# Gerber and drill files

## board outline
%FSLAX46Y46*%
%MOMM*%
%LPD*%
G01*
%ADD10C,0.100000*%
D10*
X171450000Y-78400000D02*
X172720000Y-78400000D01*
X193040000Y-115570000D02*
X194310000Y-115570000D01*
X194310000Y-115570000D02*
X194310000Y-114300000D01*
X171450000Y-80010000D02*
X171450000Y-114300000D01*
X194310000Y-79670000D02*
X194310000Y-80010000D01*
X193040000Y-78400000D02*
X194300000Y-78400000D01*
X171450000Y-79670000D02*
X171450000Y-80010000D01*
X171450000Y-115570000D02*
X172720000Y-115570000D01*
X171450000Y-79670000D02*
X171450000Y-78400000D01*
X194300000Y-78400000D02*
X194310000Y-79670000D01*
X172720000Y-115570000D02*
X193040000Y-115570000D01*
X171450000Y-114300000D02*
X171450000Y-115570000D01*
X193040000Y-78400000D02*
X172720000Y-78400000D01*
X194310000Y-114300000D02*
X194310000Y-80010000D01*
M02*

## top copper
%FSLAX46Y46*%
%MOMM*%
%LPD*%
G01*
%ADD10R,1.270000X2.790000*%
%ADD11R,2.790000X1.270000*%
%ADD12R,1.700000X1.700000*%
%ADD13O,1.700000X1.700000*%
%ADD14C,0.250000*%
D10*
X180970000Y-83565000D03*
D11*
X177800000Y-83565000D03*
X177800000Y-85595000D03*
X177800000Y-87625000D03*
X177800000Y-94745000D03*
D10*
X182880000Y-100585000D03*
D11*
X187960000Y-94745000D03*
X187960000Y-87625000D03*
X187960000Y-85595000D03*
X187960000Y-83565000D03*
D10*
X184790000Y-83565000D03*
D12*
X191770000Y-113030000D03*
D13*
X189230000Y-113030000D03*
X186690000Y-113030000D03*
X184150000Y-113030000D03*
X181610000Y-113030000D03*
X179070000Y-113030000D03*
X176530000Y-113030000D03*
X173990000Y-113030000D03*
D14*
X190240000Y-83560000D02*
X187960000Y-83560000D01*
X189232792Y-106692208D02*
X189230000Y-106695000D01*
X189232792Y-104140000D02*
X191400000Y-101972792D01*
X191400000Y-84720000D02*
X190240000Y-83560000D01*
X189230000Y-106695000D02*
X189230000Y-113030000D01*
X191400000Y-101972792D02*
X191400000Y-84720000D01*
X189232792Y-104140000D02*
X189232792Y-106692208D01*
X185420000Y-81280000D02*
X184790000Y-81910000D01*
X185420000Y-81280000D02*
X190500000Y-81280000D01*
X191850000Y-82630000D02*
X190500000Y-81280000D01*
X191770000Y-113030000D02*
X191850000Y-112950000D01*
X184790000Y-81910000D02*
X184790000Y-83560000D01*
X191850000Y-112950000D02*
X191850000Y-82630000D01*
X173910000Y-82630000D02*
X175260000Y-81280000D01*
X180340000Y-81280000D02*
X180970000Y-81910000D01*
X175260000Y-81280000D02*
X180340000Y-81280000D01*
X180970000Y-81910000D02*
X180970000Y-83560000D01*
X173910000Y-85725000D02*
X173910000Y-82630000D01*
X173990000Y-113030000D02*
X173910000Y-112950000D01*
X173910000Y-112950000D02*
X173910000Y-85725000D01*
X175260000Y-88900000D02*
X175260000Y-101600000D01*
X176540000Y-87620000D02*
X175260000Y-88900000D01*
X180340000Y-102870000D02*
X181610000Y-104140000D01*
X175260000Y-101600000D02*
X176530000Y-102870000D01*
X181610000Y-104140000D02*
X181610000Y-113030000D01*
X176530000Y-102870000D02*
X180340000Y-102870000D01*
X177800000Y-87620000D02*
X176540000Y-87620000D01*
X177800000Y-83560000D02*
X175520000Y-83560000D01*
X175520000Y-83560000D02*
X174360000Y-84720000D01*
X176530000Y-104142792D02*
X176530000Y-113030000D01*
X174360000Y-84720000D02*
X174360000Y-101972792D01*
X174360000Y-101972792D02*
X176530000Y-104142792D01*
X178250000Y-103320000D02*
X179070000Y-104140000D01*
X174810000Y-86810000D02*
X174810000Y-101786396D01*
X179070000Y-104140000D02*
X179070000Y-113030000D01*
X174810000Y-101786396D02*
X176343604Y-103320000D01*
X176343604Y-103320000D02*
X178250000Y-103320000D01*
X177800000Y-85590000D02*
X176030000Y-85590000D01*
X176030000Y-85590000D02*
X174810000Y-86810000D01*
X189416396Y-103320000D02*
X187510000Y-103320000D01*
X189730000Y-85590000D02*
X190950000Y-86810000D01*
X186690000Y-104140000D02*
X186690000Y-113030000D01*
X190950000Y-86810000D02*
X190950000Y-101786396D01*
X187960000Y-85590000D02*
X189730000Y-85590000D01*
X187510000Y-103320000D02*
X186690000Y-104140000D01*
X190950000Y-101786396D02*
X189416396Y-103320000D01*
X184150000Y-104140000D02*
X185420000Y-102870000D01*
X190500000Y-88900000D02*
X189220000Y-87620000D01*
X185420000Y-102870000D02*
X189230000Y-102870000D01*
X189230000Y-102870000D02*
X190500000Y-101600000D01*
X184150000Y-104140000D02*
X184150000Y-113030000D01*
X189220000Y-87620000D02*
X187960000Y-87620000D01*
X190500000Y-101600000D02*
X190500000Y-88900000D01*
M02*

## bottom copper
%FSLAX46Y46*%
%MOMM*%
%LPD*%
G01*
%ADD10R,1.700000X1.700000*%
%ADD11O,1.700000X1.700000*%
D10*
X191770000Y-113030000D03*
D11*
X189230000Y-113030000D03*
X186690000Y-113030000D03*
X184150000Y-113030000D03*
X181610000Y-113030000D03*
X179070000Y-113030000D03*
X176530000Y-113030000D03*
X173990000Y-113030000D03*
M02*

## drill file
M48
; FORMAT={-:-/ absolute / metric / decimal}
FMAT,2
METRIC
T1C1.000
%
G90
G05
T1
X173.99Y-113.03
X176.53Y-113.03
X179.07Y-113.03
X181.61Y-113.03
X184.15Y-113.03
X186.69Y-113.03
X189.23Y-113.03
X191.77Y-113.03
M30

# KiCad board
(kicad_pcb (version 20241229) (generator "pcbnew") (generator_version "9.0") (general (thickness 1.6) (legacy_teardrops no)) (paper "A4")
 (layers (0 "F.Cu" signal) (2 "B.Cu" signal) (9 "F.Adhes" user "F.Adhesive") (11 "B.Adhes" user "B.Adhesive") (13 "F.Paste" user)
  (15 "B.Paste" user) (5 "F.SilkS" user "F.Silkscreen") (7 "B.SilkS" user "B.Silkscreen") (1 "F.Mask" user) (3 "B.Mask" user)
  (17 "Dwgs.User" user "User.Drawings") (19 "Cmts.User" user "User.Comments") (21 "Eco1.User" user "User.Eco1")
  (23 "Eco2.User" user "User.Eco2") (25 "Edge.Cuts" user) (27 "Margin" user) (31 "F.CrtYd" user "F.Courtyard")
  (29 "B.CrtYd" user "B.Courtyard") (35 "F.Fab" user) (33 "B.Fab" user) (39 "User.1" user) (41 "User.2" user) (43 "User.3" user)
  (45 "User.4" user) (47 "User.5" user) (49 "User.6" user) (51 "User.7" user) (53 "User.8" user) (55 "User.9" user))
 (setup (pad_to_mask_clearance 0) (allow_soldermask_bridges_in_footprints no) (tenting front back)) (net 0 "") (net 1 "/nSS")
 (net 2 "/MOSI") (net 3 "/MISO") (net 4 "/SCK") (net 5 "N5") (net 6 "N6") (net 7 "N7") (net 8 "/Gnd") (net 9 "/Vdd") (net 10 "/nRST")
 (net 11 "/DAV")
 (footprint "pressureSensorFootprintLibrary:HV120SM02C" (layer "F.Cu") (at 182.88 92.075 90)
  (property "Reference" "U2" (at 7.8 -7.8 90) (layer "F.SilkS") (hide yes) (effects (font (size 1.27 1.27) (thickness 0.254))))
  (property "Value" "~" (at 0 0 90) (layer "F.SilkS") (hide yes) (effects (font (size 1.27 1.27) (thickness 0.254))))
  (pad "1" smd rect (at 8.51 -1.91 180) (size 1.27 2.79) (layers "F.Cu" "F.Mask" "F.Paste") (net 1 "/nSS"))
  (pad "2" smd rect (at 8.51 -5.08 90) (size 1.27 2.79) (layers "F.Cu" "F.Mask" "F.Paste") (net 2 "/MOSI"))
  (pad "3" smd rect (at 6.48 -5.08 90) (size 1.27 2.79) (layers "F.Cu" "F.Mask" "F.Paste") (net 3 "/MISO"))
  (pad "4" smd rect (at 4.45 -5.08 90) (size 1.27 2.79) (layers "F.Cu" "F.Mask" "F.Paste") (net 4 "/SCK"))
  (pad "5" smd rect (at -2.67 -5.08 90) (size 1.27 2.79) (layers "F.Cu" "F.Mask" "F.Paste") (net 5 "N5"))
  (pad "6" smd rect (at -8.51 0 180) (size 1.27 2.79) (layers "F.Cu" "F.Mask" "F.Paste") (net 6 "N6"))
  (pad "7" smd rect (at -2.67 5.08 90) (size 1.27 2.79) (layers "F.Cu" "F.Mask" "F.Paste") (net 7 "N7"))
  (pad "8" smd rect (at 4.45 5.08 90) (size 1.27 2.79) (layers "F.Cu" "F.Mask" "F.Paste") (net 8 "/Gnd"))
  (pad "9" smd rect (at 6.48 5.08 90) (size 1.27 2.79) (layers "F.Cu" "F.Mask" "F.Paste") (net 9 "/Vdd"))
  (pad "10" smd rect (at 8.51 5.08 90) (size 1.27 2.79) (layers "F.Cu" "F.Mask" "F.Paste") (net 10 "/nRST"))
  (pad "11" smd rect (at 8.51 1.91 180) (size 1.27 2.79) (layers "F.Cu" "F.Mask" "F.Paste") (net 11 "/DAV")))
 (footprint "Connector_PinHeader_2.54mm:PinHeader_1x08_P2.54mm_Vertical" (layer "B.Cu") (at 191.77 113.03 90)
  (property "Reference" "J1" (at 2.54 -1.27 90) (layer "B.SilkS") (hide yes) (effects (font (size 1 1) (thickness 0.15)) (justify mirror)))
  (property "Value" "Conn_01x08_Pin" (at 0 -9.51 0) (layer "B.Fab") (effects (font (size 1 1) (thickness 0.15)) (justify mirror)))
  (pad "1" thru_hole rect (at 0 0 90) (size 1.7 1.7) (drill 1) (layers "*.Cu" "*.Mask") (remove_unused_layers no) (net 11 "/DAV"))
  (pad "2" thru_hole oval (at 0 -2.54 90) (size 1.7 1.7) (drill 1) (layers "*.Cu" "*.Mask") (remove_unused_layers no) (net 10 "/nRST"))
  (pad "3" thru_hole oval (at 0 -5.08 90) (size 1.7 1.7) (drill 1) (layers "*.Cu" "*.Mask") (remove_unused_layers no) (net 9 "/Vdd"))
  (pad "4" thru_hole oval (at 0 -7.62 90) (size 1.7 1.7) (drill 1) (layers "*.Cu" "*.Mask") (remove_unused_layers no) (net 8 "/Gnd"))
  (pad "5" thru_hole oval (at 0 -10.16 90) (size 1.7 1.7) (drill 1) (layers "*.Cu" "*.Mask") (remove_unused_layers no) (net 4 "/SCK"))
  (pad "6" thru_hole oval (at 0 -12.7 90) (size 1.7 1.7) (drill 1) (layers "*.Cu" "*.Mask") (remove_unused_layers no) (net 3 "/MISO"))
  (pad "7" thru_hole oval (at 0 -15.24 90) (size 1.7 1.7) (drill 1) (layers "*.Cu" "*.Mask") (remove_unused_layers no) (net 2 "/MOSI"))
  (pad "8" thru_hole oval (at 0 -17.78 90) (size 1.7 1.7) (drill 1) (layers "*.Cu" "*.Mask") (remove_unused_layers no) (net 1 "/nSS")))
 (gr_line (start 171.45 78.4) (end 172.72 78.4) (stroke (width 0.1) (type default)) (layer "Edge.Cuts"))
 (gr_line (start 193.04 115.57) (end 194.31 115.57) (stroke (width 0.1) (type default)) (layer "Edge.Cuts"))
 (gr_line (start 194.31 115.57) (end 194.31 114.3) (stroke (width 0.1) (type default)) (layer "Edge.Cuts"))
 (gr_line (start 171.45 80.01) (end 171.45 114.3) (stroke (width 0.1) (type default)) (layer "Edge.Cuts"))
 (gr_line (start 194.31 79.67) (end 194.31 80.01) (stroke (width 0.1) (type default)) (layer "Edge.Cuts"))
 (gr_line (start 193.04 78.4) (end 194.3 78.4) (stroke (width 0.1) (type default)) (layer "Edge.Cuts"))
 (gr_line (start 171.45 79.67) (end 171.45 80.01) (stroke (width 0.1) (type default)) (layer "Edge.Cuts"))
 (gr_line (start 171.45 115.57) (end 172.72 115.57) (stroke (width 0.1) (type default)) (layer "Edge.Cuts"))
 (gr_line (start 171.45 79.67) (end 171.45 78.4) (stroke (width 0.1) (type default)) (layer "Edge.Cuts"))
 (gr_line (start 194.3 78.4) (end 194.31 79.67) (stroke (width 0.1) (type default)) (layer "Edge.Cuts"))
 (gr_line (start 172.72 115.57) (end 193.04 115.57) (stroke (width 0.1) (type default)) (layer "Edge.Cuts"))
 (gr_line (start 171.45 114.3) (end 171.45 115.57) (stroke (width 0.1) (type default)) (layer "Edge.Cuts"))
 (gr_line (start 193.04 78.4) (end 172.72 78.4) (stroke (width 0.1) (type default)) (layer "Edge.Cuts"))
 (gr_line (start 194.31 114.3) (end 194.31 80.01) (stroke (width 0.1) (type default)) (layer "Edge.Cuts"))
 (segment (start 190.24 83.56) (end 187.96 83.56) (width 0.25) (layer "F.Cu") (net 10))
 (segment (start 189.232792 106.692208) (end 189.23 106.695) (width 0.25) (layer "F.Cu") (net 10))
 (segment (start 189.232792 104.14) (end 191.4 101.972792) (width 0.25) (layer "F.Cu") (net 10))
 (segment (start 191.4 84.72) (end 190.24 83.56) (width 0.25) (layer "F.Cu") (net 10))
 (segment (start 189.23 106.695) (end 189.23 113.03) (width 0.25) (layer "F.Cu") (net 10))
 (segment (start 191.4 101.972792) (end 191.4 84.72) (width 0.25) (layer "F.Cu") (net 10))
 (segment (start 189.232792 104.14) (end 189.232792 106.692208) (width 0.25) (layer "F.Cu") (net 10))
 (segment (start 185.42 81.28) (end 184.79 81.91) (width 0.25) (layer "F.Cu") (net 11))
 (segment (start 185.42 81.28) (end 190.5 81.28) (width 0.25) (layer "F.Cu") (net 11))
 (segment (start 191.85 82.63) (end 190.5 81.28) (width 0.25) (layer "F.Cu") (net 11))
 (segment (start 191.77 113.03) (end 191.85 112.95) (width 0.25) (layer "F.Cu") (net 11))
 (segment (start 184.79 81.91) (end 184.79 83.56) (width 0.25) (layer "F.Cu") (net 11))
 (segment (start 191.85 112.95) (end 191.85 82.63) (width 0.25) (layer "F.Cu") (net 11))
 (segment (start 173.91 82.63) (end 175.26 81.28) (width 0.25) (layer "F.Cu") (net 1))
 (segment (start 180.34 81.28) (end 180.97 81.91) (width 0.25) (layer "F.Cu") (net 1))
 (segment (start 175.26 81.28) (end 180.34 81.28) (width 0.25) (layer "F.Cu") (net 1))
 (segment (start 180.97 81.91) (end 180.97 83.56) (width 0.25) (layer "F.Cu") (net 1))
 (segment (start 173.91 85.725) (end 173.91 82.63) (width 0.25) (layer "F.Cu") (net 1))
 (segment (start 173.99 113.03) (end 173.91 112.95) (width 0.25) (layer "F.Cu") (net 1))
 (segment (start 173.91 112.95) (end 173.91 85.725) (width 0.25) (layer "F.Cu") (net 1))
 (segment (start 175.26 88.9) (end 175.26 101.6) (width 0.25) (layer "F.Cu") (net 4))
 (segment (start 176.54 87.62) (end 175.26 88.9) (width 0.25) (layer "F.Cu") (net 4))
 (segment (start 180.34 102.87) (end 181.61 104.14) (width 0.25) (layer "F.Cu") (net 4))
 (segment (start 175.26 101.6) (end 176.53 102.87) (width 0.25) (layer "F.Cu") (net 4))
 (segment (start 181.61 104.14) (end 181.61 113.03) (width 0.25) (layer "F.Cu") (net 4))
 (segment (start 176.53 102.87) (end 180.34 102.87) (width 0.25) (layer "F.Cu") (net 4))
 (segment (start 177.8 87.62) (end 176.54 87.62) (width 0.25) (layer "F.Cu") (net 4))
 (segment (start 177.8 83.56) (end 175.52 83.56) (width 0.25) (layer "F.Cu") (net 2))
 (segment (start 175.52 83.56) (end 174.36 84.72) (width 0.25) (layer "F.Cu") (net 2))
 (segment (start 176.53 104.142792) (end 176.53 113.03) (width 0.25) (layer "F.Cu") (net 2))
 (segment (start 174.36 84.72) (end 174.36 101.972792) (width 0.25) (layer "F.Cu") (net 2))
 (segment (start 174.36 101.972792) (end 176.53 104.142792) (width 0.25) (layer "F.Cu") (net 2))
 (segment (start 178.25 103.32) (end 179.07 104.14) (width 0.25) (layer "F.Cu") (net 3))
 (segment (start 174.81 86.81) (end 174.81 101.786396) (width 0.25) (layer "F.Cu") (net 3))
 (segment (start 179.07 104.14) (end 179.07 113.03) (width 0.25) (layer "F.Cu") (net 3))
 (segment (start 174.81 101.786396) (end 176.343604 103.32) (width 0.25) (layer "F.Cu") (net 3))
 (segment (start 176.343604 103.32) (end 178.25 103.32) (width 0.25) (layer "F.Cu") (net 3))
 (segment (start 177.8 85.59) (end 176.03 85.59) (width 0.25) (layer "F.Cu") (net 3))
 (segment (start 176.03 85.59) (end 174.81 86.81) (width 0.25) (layer "F.Cu") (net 3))
 (segment (start 189.416396 103.32) (end 187.51 103.32) (width 0.25) (layer "F.Cu") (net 9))
 (segment (start 189.73 85.59) (end 190.95 86.81) (width 0.25) (layer "F.Cu") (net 9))
 (segment (start 186.69 104.14) (end 186.69 113.03) (width 0.25) (layer "F.Cu") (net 9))
 (segment (start 190.95 86.81) (end 190.95 101.786396) (width 0.25) (layer "F.Cu") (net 9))
 (segment (start 187.96 85.59) (end 189.73 85.59) (width 0.25) (layer "F.Cu") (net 9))
 (segment (start 187.51 103.32) (end 186.69 104.14) (width 0.25) (layer "F.Cu") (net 9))
 (segment (start 190.95 101.786396) (end 189.416396 103.32) (width 0.25) (layer "F.Cu") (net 9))
 (segment (start 184.15 104.14) (end 185.42 102.87) (width 0.25) (layer "F.Cu") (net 8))
 (segment (start 190.5 88.9) (end 189.22 87.62) (width 0.25) (layer "F.Cu") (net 8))
 (segment (start 185.42 102.87) (end 189.23 102.87) (width 0.25) (layer "F.Cu") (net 8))
 (segment (start 189.23 102.87) (end 190.5 101.6) (width 0.25) (layer "F.Cu") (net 8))
 (segment (start 184.15 104.14) (end 184.15 113.03) (width 0.25) (layer "F.Cu") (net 8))
 (segment (start 189.22 87.62) (end 187.96 87.62) (width 0.25) (layer "F.Cu") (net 8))
 (segment (start 190.5 101.6) (end 190.5 88.9) (width 0.25) (layer "F.Cu") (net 8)))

